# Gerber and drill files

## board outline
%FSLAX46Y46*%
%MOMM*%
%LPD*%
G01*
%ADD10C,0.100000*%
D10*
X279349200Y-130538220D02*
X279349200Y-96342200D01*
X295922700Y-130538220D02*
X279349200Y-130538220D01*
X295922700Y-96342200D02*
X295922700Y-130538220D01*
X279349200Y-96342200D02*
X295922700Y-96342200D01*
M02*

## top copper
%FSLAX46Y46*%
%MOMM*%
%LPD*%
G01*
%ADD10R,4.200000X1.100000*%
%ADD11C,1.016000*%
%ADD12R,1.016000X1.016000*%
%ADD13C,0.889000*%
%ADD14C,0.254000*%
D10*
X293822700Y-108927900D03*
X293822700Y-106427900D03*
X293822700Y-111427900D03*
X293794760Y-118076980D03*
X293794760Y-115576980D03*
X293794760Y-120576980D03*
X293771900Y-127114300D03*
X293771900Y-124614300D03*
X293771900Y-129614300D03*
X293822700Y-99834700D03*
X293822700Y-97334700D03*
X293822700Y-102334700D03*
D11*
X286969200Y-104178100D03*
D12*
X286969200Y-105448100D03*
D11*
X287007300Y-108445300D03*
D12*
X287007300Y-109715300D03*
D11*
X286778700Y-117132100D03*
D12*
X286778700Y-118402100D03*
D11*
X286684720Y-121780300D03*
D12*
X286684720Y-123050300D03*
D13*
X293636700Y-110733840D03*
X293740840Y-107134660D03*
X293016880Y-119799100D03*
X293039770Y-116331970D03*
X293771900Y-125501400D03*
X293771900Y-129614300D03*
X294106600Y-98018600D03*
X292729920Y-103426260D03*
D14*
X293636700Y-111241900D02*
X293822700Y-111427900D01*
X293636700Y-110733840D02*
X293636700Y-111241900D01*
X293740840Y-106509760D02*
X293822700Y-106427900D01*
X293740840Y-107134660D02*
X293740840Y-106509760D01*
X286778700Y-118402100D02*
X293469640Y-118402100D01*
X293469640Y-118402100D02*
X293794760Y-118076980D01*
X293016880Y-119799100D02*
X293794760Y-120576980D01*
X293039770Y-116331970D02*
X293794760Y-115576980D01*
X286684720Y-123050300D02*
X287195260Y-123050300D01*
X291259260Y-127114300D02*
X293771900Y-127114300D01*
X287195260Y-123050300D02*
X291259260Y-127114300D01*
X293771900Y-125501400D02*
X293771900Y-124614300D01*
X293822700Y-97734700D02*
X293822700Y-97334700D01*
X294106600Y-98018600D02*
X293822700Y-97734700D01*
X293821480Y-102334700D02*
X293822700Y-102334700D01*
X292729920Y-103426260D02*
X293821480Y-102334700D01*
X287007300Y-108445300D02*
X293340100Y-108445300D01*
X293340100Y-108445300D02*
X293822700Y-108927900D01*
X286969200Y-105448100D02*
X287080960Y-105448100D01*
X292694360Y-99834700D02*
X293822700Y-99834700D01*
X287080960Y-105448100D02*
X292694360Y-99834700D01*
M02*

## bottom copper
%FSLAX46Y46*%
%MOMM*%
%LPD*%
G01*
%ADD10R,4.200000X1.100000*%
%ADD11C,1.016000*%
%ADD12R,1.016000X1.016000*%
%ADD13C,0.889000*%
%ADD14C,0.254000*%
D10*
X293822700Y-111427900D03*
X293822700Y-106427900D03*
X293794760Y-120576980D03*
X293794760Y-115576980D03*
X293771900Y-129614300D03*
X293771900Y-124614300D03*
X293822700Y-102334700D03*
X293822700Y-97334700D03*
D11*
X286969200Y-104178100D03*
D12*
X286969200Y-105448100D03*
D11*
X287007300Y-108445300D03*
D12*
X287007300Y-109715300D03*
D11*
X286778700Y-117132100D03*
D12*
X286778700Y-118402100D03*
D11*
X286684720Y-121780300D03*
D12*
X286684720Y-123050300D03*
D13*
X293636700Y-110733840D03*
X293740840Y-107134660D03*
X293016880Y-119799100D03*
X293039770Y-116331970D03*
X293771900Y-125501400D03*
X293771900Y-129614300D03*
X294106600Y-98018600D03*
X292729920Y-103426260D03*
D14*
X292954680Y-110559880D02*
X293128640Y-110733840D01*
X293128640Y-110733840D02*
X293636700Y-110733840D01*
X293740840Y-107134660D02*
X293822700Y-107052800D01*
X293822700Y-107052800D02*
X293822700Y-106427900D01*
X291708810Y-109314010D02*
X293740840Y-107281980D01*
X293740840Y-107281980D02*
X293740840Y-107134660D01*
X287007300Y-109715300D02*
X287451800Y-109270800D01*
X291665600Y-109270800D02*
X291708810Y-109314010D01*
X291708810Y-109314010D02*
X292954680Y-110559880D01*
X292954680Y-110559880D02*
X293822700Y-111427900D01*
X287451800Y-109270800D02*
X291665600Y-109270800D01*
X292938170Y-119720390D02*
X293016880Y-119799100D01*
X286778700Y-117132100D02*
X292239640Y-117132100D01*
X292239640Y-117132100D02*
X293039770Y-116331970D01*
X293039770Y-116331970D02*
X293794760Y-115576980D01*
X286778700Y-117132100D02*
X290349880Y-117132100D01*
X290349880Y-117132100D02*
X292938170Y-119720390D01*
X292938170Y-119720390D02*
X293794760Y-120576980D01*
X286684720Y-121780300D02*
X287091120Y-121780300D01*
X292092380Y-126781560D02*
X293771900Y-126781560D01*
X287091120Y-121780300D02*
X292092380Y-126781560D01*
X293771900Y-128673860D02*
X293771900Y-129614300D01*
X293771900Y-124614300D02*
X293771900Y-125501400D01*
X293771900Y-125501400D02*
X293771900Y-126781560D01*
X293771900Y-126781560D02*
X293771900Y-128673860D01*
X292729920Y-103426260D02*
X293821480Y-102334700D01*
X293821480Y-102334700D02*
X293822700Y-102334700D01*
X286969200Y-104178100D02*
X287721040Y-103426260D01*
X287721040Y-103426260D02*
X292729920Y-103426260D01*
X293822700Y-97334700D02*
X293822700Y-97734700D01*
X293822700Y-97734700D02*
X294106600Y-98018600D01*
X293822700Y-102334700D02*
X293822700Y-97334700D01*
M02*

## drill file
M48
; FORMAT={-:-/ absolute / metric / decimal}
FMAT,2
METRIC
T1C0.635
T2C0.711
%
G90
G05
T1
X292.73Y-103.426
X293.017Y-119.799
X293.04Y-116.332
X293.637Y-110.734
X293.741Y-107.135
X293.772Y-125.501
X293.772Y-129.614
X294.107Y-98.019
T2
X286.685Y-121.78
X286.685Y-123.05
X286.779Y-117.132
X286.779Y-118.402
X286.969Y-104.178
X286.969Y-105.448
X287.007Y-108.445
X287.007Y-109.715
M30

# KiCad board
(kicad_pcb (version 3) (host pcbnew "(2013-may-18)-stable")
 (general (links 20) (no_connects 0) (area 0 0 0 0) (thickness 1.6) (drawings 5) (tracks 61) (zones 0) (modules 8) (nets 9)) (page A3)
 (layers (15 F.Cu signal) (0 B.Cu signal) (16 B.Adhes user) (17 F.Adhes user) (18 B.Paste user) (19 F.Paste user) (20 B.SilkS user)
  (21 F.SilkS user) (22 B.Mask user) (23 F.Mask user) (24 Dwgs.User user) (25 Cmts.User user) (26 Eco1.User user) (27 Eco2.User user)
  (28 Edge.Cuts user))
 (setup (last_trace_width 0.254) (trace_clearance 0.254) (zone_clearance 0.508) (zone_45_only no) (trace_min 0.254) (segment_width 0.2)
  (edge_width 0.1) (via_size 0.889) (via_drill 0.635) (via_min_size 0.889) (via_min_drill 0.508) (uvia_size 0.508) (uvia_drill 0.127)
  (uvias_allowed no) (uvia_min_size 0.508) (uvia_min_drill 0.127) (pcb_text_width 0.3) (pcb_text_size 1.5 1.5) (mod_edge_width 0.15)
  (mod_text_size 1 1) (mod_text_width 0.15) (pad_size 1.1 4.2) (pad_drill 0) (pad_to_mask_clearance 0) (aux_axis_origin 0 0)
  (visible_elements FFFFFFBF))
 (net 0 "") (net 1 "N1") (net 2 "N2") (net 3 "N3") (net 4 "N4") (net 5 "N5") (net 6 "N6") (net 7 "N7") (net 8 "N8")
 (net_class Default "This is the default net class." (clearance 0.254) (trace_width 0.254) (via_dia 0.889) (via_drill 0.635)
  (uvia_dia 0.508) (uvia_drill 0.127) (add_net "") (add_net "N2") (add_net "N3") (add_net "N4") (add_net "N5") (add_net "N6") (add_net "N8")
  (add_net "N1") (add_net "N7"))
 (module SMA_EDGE (layer F.Cu) (at 295.9227 108.9279 90)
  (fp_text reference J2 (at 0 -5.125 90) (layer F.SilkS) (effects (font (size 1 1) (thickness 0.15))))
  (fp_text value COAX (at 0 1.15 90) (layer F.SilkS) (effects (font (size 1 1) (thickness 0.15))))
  (pad 1 smd rect (at 0 -2.1 90) (size 1.1 4.2) (layers F.Cu F.Paste F.Mask) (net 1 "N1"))
  (pad 2 smd rect (at -2.5 -2.1 90) (size 1.1 4.2) (layers B.Cu F.Paste F.Mask) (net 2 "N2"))
  (pad 2 smd rect (at 2.5 -2.1 90) (size 1.1 4.2) (layers B.Cu F.Paste F.Mask) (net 2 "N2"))
  (pad 2 smd rect (at 2.5 -2.1 90) (size 1.1 4.2) (layers F.Cu F.Paste F.Mask) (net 2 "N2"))
  (pad 2 smd rect (at -2.5 -2.1 90) (size 1.1 4.2) (layers F.Cu F.Paste F.Mask) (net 2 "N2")))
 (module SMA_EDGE (layer F.Cu) (at 295.89476 118.07698 90)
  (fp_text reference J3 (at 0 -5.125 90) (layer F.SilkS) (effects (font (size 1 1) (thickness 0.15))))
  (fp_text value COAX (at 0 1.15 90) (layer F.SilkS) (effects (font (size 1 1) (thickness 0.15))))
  (pad 1 smd rect (at 0 -2.1 90) (size 1.1 4.2) (layers F.Cu F.Paste F.Mask) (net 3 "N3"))
  (pad 2 smd rect (at -2.5 -2.1 90) (size 1.1 4.2) (layers B.Cu F.Paste F.Mask) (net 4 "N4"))
  (pad 2 smd rect (at 2.5 -2.1 90) (size 1.1 4.2) (layers B.Cu F.Paste F.Mask) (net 4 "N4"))
  (pad 2 smd rect (at 2.5 -2.1 90) (size 1.1 4.2) (layers F.Cu F.Paste F.Mask) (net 4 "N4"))
  (pad 2 smd rect (at -2.5 -2.1 90) (size 1.1 4.2) (layers F.Cu F.Paste F.Mask) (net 4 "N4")))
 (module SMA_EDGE (layer F.Cu) (at 295.8719 127.1143 90)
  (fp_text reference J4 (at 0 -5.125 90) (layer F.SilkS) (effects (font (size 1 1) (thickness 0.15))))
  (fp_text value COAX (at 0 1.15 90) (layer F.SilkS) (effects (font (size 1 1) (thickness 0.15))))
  (pad 1 smd rect (at 0 -2.1 90) (size 1.1 4.2) (layers F.Cu F.Paste F.Mask) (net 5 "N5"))
  (pad 2 smd rect (at -2.5 -2.1 90) (size 1.1 4.2) (layers B.Cu F.Paste F.Mask) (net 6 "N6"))
  (pad 2 smd rect (at 2.5 -2.1 90) (size 1.1 4.2) (layers B.Cu F.Paste F.Mask) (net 6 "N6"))
  (pad 2 smd rect (at 2.5 -2.1 90) (size 1.1 4.2) (layers F.Cu F.Paste F.Mask) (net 6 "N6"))
  (pad 2 smd rect (at -2.5 -2.1 90) (size 1.1 4.2) (layers F.Cu F.Paste F.Mask) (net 6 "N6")))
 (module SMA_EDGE (layer F.Cu) (at 295.9227 99.8347 90)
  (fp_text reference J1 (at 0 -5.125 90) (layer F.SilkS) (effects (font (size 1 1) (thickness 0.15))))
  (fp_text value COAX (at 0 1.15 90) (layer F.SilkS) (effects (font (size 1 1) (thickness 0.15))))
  (pad 1 smd rect (at 0 -2.1 90) (size 1.1 4.2) (layers F.Cu F.Paste F.Mask) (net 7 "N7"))
  (pad 2 smd rect (at -2.5 -2.1 90) (size 1.1 4.2) (layers B.Cu F.Paste F.Mask) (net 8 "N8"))
  (pad 2 smd rect (at 2.5 -2.1 90) (size 1.1 4.2) (layers B.Cu F.Paste F.Mask) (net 8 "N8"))
  (pad 2 smd rect (at 2.5 -2.1 90) (size 1.1 4.2) (layers F.Cu F.Paste F.Mask) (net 8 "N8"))
  (pad 2 smd rect (at -2.5 -2.1 90) (size 1.1 4.2) (layers F.Cu F.Paste F.Mask) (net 8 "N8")))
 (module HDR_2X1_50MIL (layer F.Cu) (at 286.9692 104.8131 90)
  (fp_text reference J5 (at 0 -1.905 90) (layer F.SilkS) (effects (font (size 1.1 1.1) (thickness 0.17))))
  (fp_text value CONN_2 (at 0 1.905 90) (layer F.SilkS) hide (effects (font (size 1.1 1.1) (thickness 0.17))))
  (pad 2 thru_hole circle (at 0.635 0 180) (size 1.016 1.016) (drill 0.7112) (layers *.Cu *.Mask F.SilkS) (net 8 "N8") (zone_connect 2))
  (pad 1 thru_hole rect (at -0.635 0 90) (size 1.016 1.016) (drill 0.7112) (layers *.Cu *.Mask F.SilkS) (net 7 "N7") (zone_connect 2)))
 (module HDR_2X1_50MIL (layer F.Cu) (at 287.0073 109.0803 90)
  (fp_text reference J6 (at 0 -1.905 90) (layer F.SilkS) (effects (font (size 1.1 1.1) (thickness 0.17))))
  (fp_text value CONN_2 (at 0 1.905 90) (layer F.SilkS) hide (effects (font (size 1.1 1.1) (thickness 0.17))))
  (pad 2 thru_hole circle (at 0.635 0 180) (size 1.016 1.016) (drill 0.7112) (layers *.Cu *.Mask F.SilkS) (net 1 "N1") (zone_connect 2))
  (pad 1 thru_hole rect (at -0.635 0 90) (size 1.016 1.016) (drill 0.7112) (layers *.Cu *.Mask F.SilkS) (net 2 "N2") (zone_connect 2)))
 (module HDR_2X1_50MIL (layer F.Cu) (at 286.7787 117.7671 90)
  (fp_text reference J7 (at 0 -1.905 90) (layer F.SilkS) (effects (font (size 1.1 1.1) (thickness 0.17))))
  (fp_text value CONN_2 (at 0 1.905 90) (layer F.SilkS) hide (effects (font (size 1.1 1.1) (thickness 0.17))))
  (pad 2 thru_hole circle (at 0.635 0 180) (size 1.016 1.016) (drill 0.7112) (layers *.Cu *.Mask F.SilkS) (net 4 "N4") (zone_connect 2))
  (pad 1 thru_hole rect (at -0.635 0 90) (size 1.016 1.016) (drill 0.7112) (layers *.Cu *.Mask F.SilkS) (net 3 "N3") (zone_connect 2)))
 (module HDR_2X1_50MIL (layer F.Cu) (at 286.68472 122.4153 90)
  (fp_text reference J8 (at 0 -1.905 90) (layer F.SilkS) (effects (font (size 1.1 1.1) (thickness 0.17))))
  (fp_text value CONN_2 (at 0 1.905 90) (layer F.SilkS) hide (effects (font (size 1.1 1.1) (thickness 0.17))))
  (pad 2 thru_hole circle (at 0.635 0 180) (size 1.016 1.016) (drill 0.7112) (layers *.Cu *.Mask F.SilkS) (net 6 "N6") (zone_connect 2))
  (pad 1 thru_hole rect (at -0.635 0 90) (size 1.016 1.016) (drill 0.7112) (layers *.Cu *.Mask F.SilkS) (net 5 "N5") (zone_connect 2)))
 (gr_line (start 279.3492 130.53822) (end 279.3492 96.3422) (angle 90) (layer Edge.Cuts) (width 0.1))
 (gr_line (start 295.9227 130.53822) (end 279.3492 130.53822) (angle 90) (layer Edge.Cuts) (width 0.1))
 (gr_line (start 295.9227 96.3422) (end 295.9227 130.53822) (angle 90) (layer Edge.Cuts) (width 0.1))
 (gr_line (start 279.3492 96.3422) (end 295.9227 96.3422) (angle 90) (layer Edge.Cuts) (width 0.1))
 (segment (start 292.95468 110.55988) (end 293.12864 110.73384) (width 0.254) (layer B.Cu) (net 2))
 (segment (start 293.6367 111.2419) (end 293.8227 111.4279) (width 0.254) (layer F.Cu) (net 2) (status C00000))
 (segment (start 293.6367 110.73384) (end 293.6367 111.2419) (width 0.254) (layer F.Cu) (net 2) (status 800000))
 (via (at 293.6367 110.73384) (size 0.889) (layers F.Cu B.Cu) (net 2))
 (segment (start 293.12864 110.73384) (end 293.6367 110.73384) (width 0.254) (layer B.Cu) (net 2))
 (segment (start 293.74084 107.13466) (end 293.8227 107.0528) (width 0.254) (layer B.Cu) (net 2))
 (segment (start 293.8227 107.0528) (end 293.8227 106.4279) (width 0.254) (layer B.Cu) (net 2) (status 800000))
 (segment (start 291.70881 109.31401) (end 293.74084 107.28198) (width 0.254) (layer B.Cu) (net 2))
 (segment (start 293.74084 106.50976) (end 293.8227 106.4279) (width 0.254) (layer F.Cu) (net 2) (status C00000))
 (segment (start 293.74084 107.13466) (end 293.74084 106.50976) (width 0.254) (layer F.Cu) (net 2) (status 800000))
 (via (at 293.74084 107.13466) (size 0.889) (layers F.Cu B.Cu) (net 2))
 (segment (start 293.74084 107.28198) (end 293.74084 107.13466) (width 0.254) (layer B.Cu) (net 2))
 (segment (start 287.0073 109.7153) (end 287.4518 109.2708) (width 0.254) (layer B.Cu) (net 2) (status C00000))
 (segment (start 291.6656 109.2708) (end 291.70881 109.31401) (width 0.254) (layer B.Cu) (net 2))
 (segment (start 291.70881 109.31401) (end 292.95468 110.55988) (width 0.254) (layer B.Cu) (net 2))
 (segment (start 292.95468 110.55988) (end 293.8227 111.4279) (width 0.254) (layer B.Cu) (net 2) (status 800000))
 (segment (start 287.4518 109.2708) (end 291.6656 109.2708) (width 0.254) (layer B.Cu) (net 2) (status 400000))
 (segment (start 286.7787 118.4021) (end 293.46964 118.4021) (width 0.254) (layer F.Cu) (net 3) (status C00000))
 (segment (start 293.46964 118.4021) (end 293.79476 118.07698) (width 0.254) (layer F.Cu) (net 3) (status C00000))
 (segment (start 292.93817 119.72039) (end 293.01688 119.7991) (width 0.254) (layer B.Cu) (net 4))
 (segment (start 293.01688 119.7991) (end 293.79476 120.57698) (width 0.254) (layer F.Cu) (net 4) (status 800000))
 (via (at 293.01688 119.7991) (size 0.889) (layers F.Cu B.Cu) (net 4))
 (via (at 293.03977 116.33197) (size 0.889) (layers F.Cu B.Cu) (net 4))
 (segment (start 293.03977 116.33197) (end 293.79476 115.57698) (width 0.254) (layer F.Cu) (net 4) (status 800000))
 (segment (start 286.7787 117.1321) (end 292.23964 117.1321) (width 0.254) (layer B.Cu) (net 4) (status 400000))
 (segment (start 292.23964 117.1321) (end 293.03977 116.33197) (width 0.254) (layer B.Cu) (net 4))
 (segment (start 293.03977 116.33197) (end 293.79476 115.57698) (width 0.254) (layer B.Cu) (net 4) (status 800000))
 (segment (start 286.7787 117.1321) (end 290.34988 117.1321) (width 0.254) (layer B.Cu) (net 4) (status 400000))
 (segment (start 290.34988 117.1321) (end 292.93817 119.72039) (width 0.254) (layer B.Cu) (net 4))
 (segment (start 292.93817 119.72039) (end 293.79476 120.57698) (width 0.254) (layer B.Cu) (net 4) (status 800000))
 (segment (start 286.68472 123.0503) (end 287.19526 123.0503) (width 0.254) (layer F.Cu) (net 5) (status 400000))
 (segment (start 291.25926 127.1143) (end 293.7719 127.1143) (width 0.254) (layer F.Cu) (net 5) (status 800000))
 (segment (start 287.19526 123.0503) (end 291.25926 127.1143) (width 0.254) (layer F.Cu) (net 5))
 (via (at 293.7719 125.5014) (size 0.889) (layers F.Cu B.Cu) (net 6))
 (segment (start 293.7719 125.5014) (end 293.7719 124.6143) (width 0.254) (layer F.Cu) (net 6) (status 800000))
 (segment (start 286.68472 121.7803) (end 287.09112 121.7803) (width 0.254) (layer B.Cu) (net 6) (status C00000))
 (segment (start 292.09238 126.78156) (end 293.7719 126.78156) (width 0.254) (layer B.Cu) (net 6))
 (segment (start 287.09112 121.7803) (end 292.09238 126.78156) (width 0.254) (layer B.Cu) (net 6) (status 400000))
 (segment (start 293.7719 128.67386) (end 293.7719 129.6143) (width 0.254) (layer B.Cu) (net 6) (status 800000))
 (via (at 293.7719 129.6143) (size 0.889) (layers F.Cu B.Cu) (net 6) (status C00000))
 (segment (start 293.7719 124.6143) (end 293.7719 125.5014) (width 0.254) (layer B.Cu) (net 6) (status 400000))
 (segment (start 293.7719 125.5014) (end 293.7719 126.78156) (width 0.254) (layer B.Cu) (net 6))
 (segment (start 293.7719 126.78156) (end 293.7719 128.67386) (width 0.254) (layer B.Cu) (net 6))
 (segment (start 292.72992 103.42626) (end 293.82148 102.3347) (width 0.254) (layer B.Cu) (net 8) (status 800000))
 (segment (start 293.82148 102.3347) (end 293.8227 102.3347) (width 0.254) (layer B.Cu) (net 8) (status C00000))
 (segment (start 286.9692 104.1781) (end 287.72104 103.42626) (width 0.254) (layer B.Cu) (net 8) (status 400000))
 (segment (start 287.72104 103.42626) (end 292.72992 103.42626) (width 0.254) (layer B.Cu) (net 8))
 (segment (start 293.8227 97.3347) (end 293.8227 97.7347) (width 0.254) (layer B.Cu) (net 8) (status C00000))
 (segment (start 293.8227 97.7347) (end 293.8227 97.3347) (width 0.254) (layer F.Cu) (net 8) (status C00000))
 (segment (start 294.1066 98.0186) (end 293.8227 97.7347) (width 0.254) (layer F.Cu) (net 8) (status 800000))
 (via (at 294.1066 98.0186) (size 0.889) (layers F.Cu B.Cu) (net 8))
 (segment (start 293.8227 97.7347) (end 294.1066 98.0186) (width 0.254) (layer B.Cu) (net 8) (status 400000))
 (segment (start 293.8227 102.3347) (end 293.8227 97.3347) (width 0.254) (layer B.Cu) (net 8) (status C00000))
 (segment (start 293.82148 102.3347) (end 293.8227 102.3347) (width 0.254) (layer F.Cu) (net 8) (status C00000))
 (via (at 292.72992 103.42626) (size 0.889) (layers F.Cu B.Cu) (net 8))
 (segment (start 292.72992 103.42626) (end 293.82148 102.3347) (width 0.254) (layer F.Cu) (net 8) (status 800000))
 (segment (start 287.0073 108.4453) (end 293.3401 108.4453) (width 0.254) (layer F.Cu) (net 1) (status C00000))
 (segment (start 293.3401 108.4453) (end 293.8227 108.9279) (width 0.254) (layer F.Cu) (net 1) (status C00000))
 (segment (start 286.9692 105.4481) (end 287.08096 105.4481) (width 0.254) (layer F.Cu) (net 7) (status C00000))
 (segment (start 292.69436 99.8347) (end 293.8227 99.8347) (width 0.254) (layer F.Cu) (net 7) (status C00000))
 (segment (start 287.08096 105.4481) (end 292.69436 99.8347) (width 0.254) (layer F.Cu) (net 7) (status C00000)))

